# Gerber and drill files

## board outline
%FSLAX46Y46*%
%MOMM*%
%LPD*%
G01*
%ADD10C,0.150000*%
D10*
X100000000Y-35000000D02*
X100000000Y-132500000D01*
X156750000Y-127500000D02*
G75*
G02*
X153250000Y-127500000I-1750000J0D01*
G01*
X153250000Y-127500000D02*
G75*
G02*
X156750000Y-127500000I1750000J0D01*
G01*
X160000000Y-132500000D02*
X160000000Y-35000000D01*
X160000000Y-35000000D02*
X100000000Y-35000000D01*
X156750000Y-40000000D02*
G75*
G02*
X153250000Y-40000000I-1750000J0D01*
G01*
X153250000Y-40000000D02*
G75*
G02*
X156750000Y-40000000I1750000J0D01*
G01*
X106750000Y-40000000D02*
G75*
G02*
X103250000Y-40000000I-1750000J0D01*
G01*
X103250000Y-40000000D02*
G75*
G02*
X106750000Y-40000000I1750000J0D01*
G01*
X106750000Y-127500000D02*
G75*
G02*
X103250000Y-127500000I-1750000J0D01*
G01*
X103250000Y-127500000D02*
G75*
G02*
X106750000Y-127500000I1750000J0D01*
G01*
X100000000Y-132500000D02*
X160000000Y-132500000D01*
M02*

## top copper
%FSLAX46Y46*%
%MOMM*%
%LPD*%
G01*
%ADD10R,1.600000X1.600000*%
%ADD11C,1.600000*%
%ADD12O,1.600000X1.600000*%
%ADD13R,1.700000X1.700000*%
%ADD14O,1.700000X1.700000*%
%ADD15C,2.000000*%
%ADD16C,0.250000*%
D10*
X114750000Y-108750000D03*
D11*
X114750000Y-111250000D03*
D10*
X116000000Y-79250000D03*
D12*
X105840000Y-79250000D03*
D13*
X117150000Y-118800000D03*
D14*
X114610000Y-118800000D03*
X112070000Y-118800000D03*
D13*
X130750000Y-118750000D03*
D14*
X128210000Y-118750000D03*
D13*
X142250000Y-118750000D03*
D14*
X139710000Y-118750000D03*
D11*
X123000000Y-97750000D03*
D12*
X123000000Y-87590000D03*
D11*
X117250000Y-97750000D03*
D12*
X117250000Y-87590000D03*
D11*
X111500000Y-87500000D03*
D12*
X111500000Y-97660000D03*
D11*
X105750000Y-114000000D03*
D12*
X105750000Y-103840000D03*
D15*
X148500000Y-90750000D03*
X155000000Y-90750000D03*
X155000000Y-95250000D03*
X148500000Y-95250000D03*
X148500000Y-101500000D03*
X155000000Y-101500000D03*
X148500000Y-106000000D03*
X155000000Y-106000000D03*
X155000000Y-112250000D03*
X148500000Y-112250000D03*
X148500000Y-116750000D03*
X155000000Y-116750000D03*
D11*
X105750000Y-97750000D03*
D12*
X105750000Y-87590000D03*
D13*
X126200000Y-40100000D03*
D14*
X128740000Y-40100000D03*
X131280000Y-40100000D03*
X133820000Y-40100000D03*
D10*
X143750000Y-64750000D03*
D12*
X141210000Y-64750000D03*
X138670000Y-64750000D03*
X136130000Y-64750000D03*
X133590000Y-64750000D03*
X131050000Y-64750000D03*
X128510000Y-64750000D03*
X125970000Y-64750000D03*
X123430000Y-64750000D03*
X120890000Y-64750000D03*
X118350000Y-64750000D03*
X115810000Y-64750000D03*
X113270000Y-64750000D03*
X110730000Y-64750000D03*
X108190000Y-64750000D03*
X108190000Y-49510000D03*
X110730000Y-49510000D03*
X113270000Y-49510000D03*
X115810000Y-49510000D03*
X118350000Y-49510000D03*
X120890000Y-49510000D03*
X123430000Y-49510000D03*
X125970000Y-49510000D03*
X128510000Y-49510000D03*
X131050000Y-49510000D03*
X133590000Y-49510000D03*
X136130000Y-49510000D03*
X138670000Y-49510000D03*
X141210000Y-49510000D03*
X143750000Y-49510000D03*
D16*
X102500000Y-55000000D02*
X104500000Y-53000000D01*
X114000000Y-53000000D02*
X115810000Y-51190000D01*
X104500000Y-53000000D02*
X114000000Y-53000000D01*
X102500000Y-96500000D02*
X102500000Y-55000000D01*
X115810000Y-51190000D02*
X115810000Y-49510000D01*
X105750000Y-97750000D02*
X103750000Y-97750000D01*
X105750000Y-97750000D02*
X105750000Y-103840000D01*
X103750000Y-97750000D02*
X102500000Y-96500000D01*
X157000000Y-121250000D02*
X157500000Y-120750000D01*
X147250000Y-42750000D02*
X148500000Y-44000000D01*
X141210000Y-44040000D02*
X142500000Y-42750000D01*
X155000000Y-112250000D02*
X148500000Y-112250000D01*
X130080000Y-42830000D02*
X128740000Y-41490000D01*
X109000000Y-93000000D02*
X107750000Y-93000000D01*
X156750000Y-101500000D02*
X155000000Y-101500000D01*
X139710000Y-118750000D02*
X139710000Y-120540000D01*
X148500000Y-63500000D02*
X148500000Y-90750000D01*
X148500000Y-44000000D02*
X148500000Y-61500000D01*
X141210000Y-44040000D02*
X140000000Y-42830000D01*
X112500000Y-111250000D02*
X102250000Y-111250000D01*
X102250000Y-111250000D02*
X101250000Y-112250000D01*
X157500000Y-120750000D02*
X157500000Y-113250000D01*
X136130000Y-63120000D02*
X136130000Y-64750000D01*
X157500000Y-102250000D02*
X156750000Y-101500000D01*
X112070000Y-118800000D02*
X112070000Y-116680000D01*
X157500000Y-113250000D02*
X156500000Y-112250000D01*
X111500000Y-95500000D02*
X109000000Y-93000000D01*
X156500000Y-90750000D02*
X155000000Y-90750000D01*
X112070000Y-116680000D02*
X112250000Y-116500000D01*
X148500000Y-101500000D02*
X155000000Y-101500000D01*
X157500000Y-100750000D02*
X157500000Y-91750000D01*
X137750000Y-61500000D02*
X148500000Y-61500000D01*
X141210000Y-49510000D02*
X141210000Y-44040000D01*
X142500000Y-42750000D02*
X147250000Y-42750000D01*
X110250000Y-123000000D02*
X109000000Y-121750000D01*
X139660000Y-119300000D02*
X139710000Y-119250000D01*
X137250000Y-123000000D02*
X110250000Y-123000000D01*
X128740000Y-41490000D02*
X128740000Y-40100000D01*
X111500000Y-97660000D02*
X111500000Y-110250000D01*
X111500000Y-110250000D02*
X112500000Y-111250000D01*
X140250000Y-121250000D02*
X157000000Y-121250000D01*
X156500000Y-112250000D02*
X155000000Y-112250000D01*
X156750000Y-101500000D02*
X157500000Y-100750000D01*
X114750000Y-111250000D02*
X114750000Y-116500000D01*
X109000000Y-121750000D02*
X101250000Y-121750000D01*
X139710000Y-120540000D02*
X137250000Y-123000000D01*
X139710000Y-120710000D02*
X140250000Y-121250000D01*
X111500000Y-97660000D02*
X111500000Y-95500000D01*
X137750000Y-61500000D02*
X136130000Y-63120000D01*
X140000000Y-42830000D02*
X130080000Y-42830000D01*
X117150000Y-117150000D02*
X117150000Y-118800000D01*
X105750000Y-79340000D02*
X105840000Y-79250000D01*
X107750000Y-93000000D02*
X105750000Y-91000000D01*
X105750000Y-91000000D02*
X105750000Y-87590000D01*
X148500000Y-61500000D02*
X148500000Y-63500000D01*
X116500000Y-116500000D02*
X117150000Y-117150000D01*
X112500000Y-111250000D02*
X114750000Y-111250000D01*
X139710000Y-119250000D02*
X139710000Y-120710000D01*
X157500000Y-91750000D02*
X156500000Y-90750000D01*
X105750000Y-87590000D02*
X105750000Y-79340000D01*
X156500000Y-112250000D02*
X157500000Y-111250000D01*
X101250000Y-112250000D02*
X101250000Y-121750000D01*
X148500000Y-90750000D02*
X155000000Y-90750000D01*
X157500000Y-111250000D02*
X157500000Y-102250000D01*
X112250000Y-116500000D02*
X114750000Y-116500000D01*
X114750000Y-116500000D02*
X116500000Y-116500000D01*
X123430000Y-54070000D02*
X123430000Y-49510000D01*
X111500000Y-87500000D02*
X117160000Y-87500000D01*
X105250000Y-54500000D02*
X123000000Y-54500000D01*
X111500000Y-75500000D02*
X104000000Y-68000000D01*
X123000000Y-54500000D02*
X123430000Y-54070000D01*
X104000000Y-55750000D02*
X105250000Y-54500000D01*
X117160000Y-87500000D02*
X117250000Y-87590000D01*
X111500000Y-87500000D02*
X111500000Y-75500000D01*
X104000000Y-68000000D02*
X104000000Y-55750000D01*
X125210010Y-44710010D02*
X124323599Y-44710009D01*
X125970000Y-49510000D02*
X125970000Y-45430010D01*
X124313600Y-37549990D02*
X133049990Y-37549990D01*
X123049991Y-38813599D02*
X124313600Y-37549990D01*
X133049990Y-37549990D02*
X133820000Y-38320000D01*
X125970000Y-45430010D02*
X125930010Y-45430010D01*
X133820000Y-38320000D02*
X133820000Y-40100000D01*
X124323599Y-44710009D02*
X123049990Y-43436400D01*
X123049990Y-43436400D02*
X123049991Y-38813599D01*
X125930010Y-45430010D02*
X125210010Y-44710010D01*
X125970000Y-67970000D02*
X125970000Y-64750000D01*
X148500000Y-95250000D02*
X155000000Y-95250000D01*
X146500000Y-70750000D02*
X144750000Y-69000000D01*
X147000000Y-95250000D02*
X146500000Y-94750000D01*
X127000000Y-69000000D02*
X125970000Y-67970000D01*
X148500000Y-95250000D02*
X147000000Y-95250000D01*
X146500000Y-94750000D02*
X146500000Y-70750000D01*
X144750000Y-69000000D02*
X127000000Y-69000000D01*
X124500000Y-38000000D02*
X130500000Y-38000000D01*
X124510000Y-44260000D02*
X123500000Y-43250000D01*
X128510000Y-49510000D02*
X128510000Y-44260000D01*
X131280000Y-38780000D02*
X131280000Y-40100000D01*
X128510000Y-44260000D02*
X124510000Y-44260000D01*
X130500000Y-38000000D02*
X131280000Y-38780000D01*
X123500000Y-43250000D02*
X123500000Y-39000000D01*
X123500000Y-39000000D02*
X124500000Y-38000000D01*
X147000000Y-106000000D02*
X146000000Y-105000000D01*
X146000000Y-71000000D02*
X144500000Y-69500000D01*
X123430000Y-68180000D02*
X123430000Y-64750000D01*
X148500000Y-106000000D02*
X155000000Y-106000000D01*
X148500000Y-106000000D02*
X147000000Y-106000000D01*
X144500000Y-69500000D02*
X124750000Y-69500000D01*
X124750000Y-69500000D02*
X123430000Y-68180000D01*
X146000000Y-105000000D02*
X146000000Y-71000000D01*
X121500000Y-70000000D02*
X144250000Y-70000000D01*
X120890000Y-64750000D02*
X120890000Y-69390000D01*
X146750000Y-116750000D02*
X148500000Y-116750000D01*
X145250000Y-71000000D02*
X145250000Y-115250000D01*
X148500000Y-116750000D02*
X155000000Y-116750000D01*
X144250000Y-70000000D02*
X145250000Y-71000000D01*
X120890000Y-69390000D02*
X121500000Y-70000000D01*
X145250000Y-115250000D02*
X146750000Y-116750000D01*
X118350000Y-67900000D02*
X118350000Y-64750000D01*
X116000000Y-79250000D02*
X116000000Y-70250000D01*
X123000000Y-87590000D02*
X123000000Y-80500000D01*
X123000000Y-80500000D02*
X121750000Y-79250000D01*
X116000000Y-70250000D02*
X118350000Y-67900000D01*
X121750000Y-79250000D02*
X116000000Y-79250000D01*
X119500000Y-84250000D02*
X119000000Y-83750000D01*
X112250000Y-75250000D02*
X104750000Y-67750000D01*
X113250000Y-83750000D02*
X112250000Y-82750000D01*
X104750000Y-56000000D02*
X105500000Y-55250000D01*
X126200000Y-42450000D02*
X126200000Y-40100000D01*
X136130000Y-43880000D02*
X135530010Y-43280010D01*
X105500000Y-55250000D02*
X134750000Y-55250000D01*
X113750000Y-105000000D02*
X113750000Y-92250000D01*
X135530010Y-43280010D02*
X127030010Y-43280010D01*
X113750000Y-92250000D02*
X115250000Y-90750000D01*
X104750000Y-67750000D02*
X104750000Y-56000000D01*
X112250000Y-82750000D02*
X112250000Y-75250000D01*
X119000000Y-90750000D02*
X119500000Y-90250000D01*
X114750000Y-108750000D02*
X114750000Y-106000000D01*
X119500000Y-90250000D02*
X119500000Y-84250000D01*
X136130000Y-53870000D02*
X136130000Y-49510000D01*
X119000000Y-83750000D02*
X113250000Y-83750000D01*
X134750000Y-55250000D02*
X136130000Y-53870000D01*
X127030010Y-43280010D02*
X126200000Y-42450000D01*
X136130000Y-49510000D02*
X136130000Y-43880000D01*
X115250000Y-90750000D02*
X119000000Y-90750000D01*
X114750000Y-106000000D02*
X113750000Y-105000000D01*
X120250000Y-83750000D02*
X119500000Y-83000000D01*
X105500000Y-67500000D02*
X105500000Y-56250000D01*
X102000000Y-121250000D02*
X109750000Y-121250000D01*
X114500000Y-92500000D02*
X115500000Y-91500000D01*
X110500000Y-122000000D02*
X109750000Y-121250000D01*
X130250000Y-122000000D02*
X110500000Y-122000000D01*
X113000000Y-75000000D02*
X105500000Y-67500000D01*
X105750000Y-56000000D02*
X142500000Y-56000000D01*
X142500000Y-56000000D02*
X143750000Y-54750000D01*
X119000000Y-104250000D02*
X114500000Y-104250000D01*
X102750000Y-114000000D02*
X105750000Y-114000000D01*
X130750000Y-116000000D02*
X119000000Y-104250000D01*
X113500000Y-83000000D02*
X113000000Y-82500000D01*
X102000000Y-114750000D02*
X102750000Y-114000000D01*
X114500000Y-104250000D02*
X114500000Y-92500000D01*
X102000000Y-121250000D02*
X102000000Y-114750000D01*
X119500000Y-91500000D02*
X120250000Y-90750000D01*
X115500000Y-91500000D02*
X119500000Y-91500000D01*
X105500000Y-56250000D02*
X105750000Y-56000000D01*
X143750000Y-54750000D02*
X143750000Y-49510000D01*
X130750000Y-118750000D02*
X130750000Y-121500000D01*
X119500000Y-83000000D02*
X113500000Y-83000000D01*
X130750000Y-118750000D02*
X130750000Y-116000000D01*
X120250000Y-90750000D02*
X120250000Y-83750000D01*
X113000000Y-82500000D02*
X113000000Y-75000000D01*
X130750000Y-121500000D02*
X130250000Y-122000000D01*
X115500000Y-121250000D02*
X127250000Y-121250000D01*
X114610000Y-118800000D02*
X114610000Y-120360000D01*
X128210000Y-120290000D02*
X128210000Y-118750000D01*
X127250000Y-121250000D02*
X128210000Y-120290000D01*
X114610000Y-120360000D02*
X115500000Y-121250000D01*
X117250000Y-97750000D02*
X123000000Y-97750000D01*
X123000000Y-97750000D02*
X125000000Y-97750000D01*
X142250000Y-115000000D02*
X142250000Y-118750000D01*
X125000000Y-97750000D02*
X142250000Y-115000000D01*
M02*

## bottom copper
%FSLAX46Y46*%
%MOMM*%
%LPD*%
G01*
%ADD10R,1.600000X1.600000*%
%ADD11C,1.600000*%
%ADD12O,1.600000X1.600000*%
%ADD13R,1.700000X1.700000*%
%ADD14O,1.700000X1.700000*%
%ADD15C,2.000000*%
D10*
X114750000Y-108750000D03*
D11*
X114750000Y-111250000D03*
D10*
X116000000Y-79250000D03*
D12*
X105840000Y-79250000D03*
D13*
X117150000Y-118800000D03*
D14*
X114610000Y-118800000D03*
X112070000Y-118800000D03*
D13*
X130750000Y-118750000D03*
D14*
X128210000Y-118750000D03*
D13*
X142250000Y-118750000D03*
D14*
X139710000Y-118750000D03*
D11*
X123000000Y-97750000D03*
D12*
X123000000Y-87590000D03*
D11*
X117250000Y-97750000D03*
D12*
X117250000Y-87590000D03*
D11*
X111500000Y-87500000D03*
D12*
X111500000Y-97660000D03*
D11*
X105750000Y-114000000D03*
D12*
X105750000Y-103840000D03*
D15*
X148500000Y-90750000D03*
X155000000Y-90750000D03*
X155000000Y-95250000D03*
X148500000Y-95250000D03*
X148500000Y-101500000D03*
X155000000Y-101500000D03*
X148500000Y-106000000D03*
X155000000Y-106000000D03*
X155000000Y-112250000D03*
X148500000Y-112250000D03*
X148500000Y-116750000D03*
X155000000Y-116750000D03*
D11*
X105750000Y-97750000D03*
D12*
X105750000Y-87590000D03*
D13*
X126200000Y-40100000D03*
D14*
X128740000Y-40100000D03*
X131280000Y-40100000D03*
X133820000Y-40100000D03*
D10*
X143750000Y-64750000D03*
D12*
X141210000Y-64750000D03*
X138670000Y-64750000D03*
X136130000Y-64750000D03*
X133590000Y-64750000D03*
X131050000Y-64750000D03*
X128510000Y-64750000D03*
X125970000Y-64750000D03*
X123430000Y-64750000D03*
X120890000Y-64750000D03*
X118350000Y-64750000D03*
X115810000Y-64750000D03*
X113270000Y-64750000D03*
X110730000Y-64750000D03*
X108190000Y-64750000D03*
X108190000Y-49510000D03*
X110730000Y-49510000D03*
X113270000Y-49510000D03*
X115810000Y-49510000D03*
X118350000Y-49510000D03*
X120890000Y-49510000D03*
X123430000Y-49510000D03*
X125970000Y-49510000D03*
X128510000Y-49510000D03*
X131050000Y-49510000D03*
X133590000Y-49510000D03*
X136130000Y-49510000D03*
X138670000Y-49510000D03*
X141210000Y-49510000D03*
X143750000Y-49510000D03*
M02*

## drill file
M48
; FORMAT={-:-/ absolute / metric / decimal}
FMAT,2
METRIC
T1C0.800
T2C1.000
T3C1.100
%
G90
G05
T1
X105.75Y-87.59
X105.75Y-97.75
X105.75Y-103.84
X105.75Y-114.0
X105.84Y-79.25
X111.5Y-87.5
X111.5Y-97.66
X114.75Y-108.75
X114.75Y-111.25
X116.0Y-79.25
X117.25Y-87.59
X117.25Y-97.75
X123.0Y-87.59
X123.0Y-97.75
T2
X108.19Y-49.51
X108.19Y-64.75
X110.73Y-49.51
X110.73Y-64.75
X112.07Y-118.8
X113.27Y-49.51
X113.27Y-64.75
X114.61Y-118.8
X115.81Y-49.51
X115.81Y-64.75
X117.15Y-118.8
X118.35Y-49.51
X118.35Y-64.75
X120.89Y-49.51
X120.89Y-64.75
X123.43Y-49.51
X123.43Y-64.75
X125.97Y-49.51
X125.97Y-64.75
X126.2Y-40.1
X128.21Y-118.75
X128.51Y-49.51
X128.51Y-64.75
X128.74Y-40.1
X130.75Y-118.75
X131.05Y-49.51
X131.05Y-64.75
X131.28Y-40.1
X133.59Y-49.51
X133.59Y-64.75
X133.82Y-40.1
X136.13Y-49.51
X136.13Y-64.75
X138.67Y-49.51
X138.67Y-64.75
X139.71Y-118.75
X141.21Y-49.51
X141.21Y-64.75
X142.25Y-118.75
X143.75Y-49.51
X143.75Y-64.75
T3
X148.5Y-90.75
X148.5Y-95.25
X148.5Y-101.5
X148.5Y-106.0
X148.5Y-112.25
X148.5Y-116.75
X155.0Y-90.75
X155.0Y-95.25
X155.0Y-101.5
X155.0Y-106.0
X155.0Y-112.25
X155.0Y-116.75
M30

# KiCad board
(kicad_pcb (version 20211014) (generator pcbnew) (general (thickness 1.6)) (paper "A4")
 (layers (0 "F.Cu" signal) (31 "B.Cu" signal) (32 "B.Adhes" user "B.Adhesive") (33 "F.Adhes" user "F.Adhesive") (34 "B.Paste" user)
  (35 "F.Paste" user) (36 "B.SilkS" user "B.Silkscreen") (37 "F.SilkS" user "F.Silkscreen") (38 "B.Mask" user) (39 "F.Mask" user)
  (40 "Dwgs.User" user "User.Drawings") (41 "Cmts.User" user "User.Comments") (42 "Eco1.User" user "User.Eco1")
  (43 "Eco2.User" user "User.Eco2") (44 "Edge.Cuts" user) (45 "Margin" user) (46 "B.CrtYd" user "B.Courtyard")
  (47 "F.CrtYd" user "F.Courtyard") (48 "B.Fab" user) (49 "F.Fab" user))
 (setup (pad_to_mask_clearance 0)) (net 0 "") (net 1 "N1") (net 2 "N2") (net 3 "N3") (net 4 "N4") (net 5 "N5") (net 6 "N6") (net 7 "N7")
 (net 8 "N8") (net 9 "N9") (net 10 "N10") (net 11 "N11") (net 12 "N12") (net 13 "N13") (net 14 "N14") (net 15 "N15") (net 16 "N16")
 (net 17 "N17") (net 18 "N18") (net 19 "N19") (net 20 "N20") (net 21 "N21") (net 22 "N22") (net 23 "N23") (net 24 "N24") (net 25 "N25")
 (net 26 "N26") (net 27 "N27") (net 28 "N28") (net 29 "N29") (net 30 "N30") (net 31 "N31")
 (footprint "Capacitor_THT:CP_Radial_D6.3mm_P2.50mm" (layer "F.Cu") (at 114.75 108.75 -90)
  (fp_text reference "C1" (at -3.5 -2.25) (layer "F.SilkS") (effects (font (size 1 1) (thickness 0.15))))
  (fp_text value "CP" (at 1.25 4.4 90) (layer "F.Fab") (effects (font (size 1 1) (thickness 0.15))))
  (pad "1" thru_hole rect locked (at 0 0 270) (size 1.6 1.6) (drill 0.8) (layers *.Cu *.Mask) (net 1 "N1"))
  (pad "2" thru_hole circle locked (at 2.5 0 270) (size 1.6 1.6) (drill 0.8) (layers *.Cu *.Mask) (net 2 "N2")))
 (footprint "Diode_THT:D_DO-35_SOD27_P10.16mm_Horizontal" (layer "F.Cu") (at 116 79.25 180)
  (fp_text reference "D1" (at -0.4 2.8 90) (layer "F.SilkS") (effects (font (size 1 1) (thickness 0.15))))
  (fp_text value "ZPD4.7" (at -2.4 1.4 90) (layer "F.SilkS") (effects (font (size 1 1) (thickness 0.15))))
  (pad "1" thru_hole rect locked (at 0 0 180) (size 1.6 1.6) (drill 0.8) (layers *.Cu *.Mask) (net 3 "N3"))
  (pad "2" thru_hole oval locked (at 10.16 0 180) (size 1.6 1.6) (drill 0.8) (layers *.Cu *.Mask) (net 2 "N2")))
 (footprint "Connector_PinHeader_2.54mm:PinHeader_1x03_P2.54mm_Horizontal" (layer "F.Cu") (at 117.15 118.8 -90)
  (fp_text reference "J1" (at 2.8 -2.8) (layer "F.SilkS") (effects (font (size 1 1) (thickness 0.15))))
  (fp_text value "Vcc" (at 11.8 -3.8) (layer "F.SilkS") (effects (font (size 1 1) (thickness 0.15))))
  (pad "1" thru_hole rect locked (at 0 0 270) (size 1.7 1.7) (drill 1) (layers *.Cu *.Mask) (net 2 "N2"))
  (pad "2" thru_hole oval locked (at 0 2.54 270) (size 1.7 1.7) (drill 1) (layers *.Cu *.Mask) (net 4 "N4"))
  (pad "3" thru_hole oval locked (at 0 5.08 270) (size 1.7 1.7) (drill 1) (layers *.Cu *.Mask) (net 2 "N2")))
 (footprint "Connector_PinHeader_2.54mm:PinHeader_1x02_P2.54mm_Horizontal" (layer "F.Cu") (at 130.75 118.75 -90)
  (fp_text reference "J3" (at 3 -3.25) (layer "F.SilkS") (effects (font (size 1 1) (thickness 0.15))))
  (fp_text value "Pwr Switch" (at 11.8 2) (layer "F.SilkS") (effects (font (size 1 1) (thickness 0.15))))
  (pad "1" thru_hole rect locked (at 0 0 270) (size 1.7 1.7) (drill 1) (layers *.Cu *.Mask) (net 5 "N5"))
  (pad "2" thru_hole oval locked (at 0 2.54 270) (size 1.7 1.7) (drill 1) (layers *.Cu *.Mask) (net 4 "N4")))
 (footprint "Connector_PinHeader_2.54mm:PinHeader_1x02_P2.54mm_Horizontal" (layer "F.Cu") (at 142.25 118.75 -90)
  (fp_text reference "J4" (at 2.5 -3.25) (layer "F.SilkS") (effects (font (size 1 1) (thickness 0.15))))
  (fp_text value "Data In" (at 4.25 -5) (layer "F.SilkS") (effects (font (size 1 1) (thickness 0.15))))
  (pad "1" thru_hole rect locked (at 0 0 270) (size 1.7 1.7) (drill 1) (layers *.Cu *.Mask) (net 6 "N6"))
  (pad "2" thru_hole oval locked (at 0 2.54 270) (size 1.7 1.7) (drill 1) (layers *.Cu *.Mask) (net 2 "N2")))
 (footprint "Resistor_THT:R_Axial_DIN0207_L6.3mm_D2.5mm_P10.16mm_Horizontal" (layer "F.Cu") (at 123 97.75 90)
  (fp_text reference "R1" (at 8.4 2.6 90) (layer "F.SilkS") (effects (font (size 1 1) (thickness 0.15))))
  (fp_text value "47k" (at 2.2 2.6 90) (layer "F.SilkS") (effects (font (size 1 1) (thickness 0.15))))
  (pad "1" thru_hole circle locked (at 0 0 90) (size 1.6 1.6) (drill 0.8) (layers *.Cu *.Mask) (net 6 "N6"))
  (pad "2" thru_hole oval locked (at 10.16 0 90) (size 1.6 1.6) (drill 0.8) (layers *.Cu *.Mask) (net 3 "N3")))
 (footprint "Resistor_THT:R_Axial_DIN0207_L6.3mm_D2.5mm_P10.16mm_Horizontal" (layer "F.Cu") (at 117.25 97.75 90)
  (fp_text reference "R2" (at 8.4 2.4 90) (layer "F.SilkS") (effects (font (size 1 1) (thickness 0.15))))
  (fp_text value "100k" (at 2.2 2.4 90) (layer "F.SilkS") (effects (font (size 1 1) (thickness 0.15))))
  (pad "1" thru_hole circle locked (at 0 0 90) (size 1.6 1.6) (drill 0.8) (layers *.Cu *.Mask) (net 6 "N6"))
  (pad "2" thru_hole oval locked (at 10.16 0 90) (size 1.6 1.6) (drill 0.8) (layers *.Cu *.Mask) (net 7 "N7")))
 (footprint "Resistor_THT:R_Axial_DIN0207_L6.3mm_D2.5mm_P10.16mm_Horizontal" (layer "F.Cu") (at 111.5 87.5 -90)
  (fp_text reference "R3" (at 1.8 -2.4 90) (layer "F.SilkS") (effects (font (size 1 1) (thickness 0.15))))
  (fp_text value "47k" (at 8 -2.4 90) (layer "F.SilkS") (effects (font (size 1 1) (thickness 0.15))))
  (pad "1" thru_hole circle locked (at 0 0 270) (size 1.6 1.6) (drill 0.8) (layers *.Cu *.Mask) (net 7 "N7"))
  (pad "2" thru_hole oval locked (at 10.16 0 270) (size 1.6 1.6) (drill 0.8) (layers *.Cu *.Mask) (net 2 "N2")))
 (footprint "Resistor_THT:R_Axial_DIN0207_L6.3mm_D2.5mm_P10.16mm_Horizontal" (layer "F.Cu") (at 105.75 114 90)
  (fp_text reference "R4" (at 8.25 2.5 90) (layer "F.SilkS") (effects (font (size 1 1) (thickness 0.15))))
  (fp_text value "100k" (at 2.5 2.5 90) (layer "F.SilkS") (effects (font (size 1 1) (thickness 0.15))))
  (pad "1" thru_hole circle locked (at 0 0 90) (size 1.6 1.6) (drill 0.8) (layers *.Cu *.Mask) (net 5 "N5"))
  (pad "2" thru_hole oval locked (at 10.16 0 90) (size 1.6 1.6) (drill 0.8) (layers *.Cu *.Mask) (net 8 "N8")))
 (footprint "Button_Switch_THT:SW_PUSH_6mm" (layer "F.Cu") (at 148.5 90.75)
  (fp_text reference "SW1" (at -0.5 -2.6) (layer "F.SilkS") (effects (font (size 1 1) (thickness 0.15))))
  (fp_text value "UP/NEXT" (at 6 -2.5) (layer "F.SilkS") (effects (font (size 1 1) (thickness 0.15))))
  (pad "1" thru_hole circle locked (at 0 0 90) (size 2 2) (drill 1.1) (layers *.Cu *.Mask) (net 2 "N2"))
  (pad "1" thru_hole circle locked (at 6.5 0 90) (size 2 2) (drill 1.1) (layers *.Cu *.Mask) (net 2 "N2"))
  (pad "2" thru_hole circle locked (at 6.5 4.5 90) (size 2 2) (drill 1.1) (layers *.Cu *.Mask) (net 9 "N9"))
  (pad "2" thru_hole circle locked (at 0 4.5 90) (size 2 2) (drill 1.1) (layers *.Cu *.Mask) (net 9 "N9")))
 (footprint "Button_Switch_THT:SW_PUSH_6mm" (layer "F.Cu") (at 148.5 101.5)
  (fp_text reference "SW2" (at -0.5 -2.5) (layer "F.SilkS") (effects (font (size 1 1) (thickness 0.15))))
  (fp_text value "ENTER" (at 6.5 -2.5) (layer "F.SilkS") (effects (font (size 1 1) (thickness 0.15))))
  (pad "1" thru_hole circle locked (at 0 0 90) (size 2 2) (drill 1.1) (layers *.Cu *.Mask) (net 2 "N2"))
  (pad "1" thru_hole circle locked (at 6.5 0 90) (size 2 2) (drill 1.1) (layers *.Cu *.Mask) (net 2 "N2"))
  (pad "2" thru_hole circle locked (at 0 4.5 90) (size 2 2) (drill 1.1) (layers *.Cu *.Mask) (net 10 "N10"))
  (pad "2" thru_hole circle locked (at 6.5 4.5 90) (size 2 2) (drill 1.1) (layers *.Cu *.Mask) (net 10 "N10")))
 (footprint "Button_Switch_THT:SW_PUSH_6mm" (layer "F.Cu") (at 148.5 112.25)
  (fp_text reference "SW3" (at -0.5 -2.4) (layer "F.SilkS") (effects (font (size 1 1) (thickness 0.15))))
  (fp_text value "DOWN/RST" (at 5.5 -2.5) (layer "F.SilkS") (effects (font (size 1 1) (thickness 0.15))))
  (pad "1" thru_hole circle locked (at 6.5 0 90) (size 2 2) (drill 1.1) (layers *.Cu *.Mask) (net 2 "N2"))
  (pad "1" thru_hole circle locked (at 0 0 90) (size 2 2) (drill 1.1) (layers *.Cu *.Mask) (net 2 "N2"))
  (pad "2" thru_hole circle locked (at 0 4.5 90) (size 2 2) (drill 1.1) (layers *.Cu *.Mask) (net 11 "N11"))
  (pad "2" thru_hole circle locked (at 6.5 4.5 90) (size 2 2) (drill 1.1) (layers *.Cu *.Mask) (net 11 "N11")))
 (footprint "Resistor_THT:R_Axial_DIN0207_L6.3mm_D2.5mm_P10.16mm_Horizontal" (layer "F.Cu") (at 105.75 97.75 90)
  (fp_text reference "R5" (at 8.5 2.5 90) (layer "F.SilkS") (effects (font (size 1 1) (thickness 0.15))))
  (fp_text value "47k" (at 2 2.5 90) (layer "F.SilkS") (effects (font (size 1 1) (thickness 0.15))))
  (pad "1" thru_hole circle locked (at 0 0 90) (size 1.6 1.6) (drill 0.8) (layers *.Cu *.Mask) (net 8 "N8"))
  (pad "2" thru_hole oval locked (at 10.16 0 90) (size 1.6 1.6) (drill 0.8) (layers *.Cu *.Mask) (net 2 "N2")))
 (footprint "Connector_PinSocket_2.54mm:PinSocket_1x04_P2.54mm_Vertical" (layer "F.Cu") (at 126.2 40.1 90)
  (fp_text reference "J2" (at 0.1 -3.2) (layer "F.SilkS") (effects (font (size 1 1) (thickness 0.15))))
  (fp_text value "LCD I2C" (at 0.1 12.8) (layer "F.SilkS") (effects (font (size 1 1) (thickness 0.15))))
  (pad "1" thru_hole rect locked (at 0 0 90) (size 1.7 1.7) (drill 1) (layers *.Cu *.Mask) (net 1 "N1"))
  (pad "2" thru_hole oval locked (at 0 2.54 90) (size 1.7 1.7) (drill 1) (layers *.Cu *.Mask) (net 2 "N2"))
  (pad "3" thru_hole oval locked (at 0 5.08 90) (size 1.7 1.7) (drill 1) (layers *.Cu *.Mask) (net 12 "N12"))
  (pad "4" thru_hole oval locked (at 0 7.62 90) (size 1.7 1.7) (drill 1) (layers *.Cu *.Mask) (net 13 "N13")))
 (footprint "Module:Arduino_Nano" (layer "B.Cu") (at 143.75 64.75 90)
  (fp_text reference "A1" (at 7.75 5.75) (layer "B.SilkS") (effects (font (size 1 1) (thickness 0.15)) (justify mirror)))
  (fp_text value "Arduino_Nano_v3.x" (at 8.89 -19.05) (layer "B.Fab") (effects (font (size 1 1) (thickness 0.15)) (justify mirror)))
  (pad "1" thru_hole rect locked (at 0 0 90) (size 1.6 1.6) (drill 1) (layers *.Cu *.Mask) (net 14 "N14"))
  (pad "2" thru_hole oval locked (at 0 -2.54 90) (size 1.6 1.6) (drill 1) (layers *.Cu *.Mask) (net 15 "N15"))
  (pad "3" thru_hole oval locked (at 0 -5.08 90) (size 1.6 1.6) (drill 1) (layers *.Cu *.Mask) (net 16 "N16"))
  (pad "4" thru_hole oval locked (at 0 -7.62 90) (size 1.6 1.6) (drill 1) (layers *.Cu *.Mask) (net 2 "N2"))
  (pad "5" thru_hole oval locked (at 0 -10.16 90) (size 1.6 1.6) (drill 1) (layers *.Cu *.Mask) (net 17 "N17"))
  (pad "6" thru_hole oval locked (at 0 -12.7 90) (size 1.6 1.6) (drill 1) (layers *.Cu *.Mask) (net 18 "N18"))
  (pad "7" thru_hole oval locked (at 0 -15.24 90) (size 1.6 1.6) (drill 1) (layers *.Cu *.Mask) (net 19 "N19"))
  (pad "8" thru_hole oval locked (at 0 -17.78 90) (size 1.6 1.6) (drill 1) (layers *.Cu *.Mask) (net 9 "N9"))
  (pad "9" thru_hole oval locked (at 0 -20.32 90) (size 1.6 1.6) (drill 1) (layers *.Cu *.Mask) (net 10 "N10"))
  (pad "10" thru_hole oval locked (at 0 -22.86 90) (size 1.6 1.6) (drill 1) (layers *.Cu *.Mask) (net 11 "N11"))
  (pad "11" thru_hole oval locked (at 0 -25.4 90) (size 1.6 1.6) (drill 1) (layers *.Cu *.Mask) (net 3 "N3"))
  (pad "12" thru_hole oval locked (at 0 -27.94 90) (size 1.6 1.6) (drill 1) (layers *.Cu *.Mask) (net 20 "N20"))
  (pad "13" thru_hole oval locked (at 0 -30.48 90) (size 1.6 1.6) (drill 1) (layers *.Cu *.Mask) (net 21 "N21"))
  (pad "14" thru_hole oval locked (at 0 -33.02 90) (size 1.6 1.6) (drill 1) (layers *.Cu *.Mask) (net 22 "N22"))
  (pad "15" thru_hole oval locked (at 0 -35.56 90) (size 1.6 1.6) (drill 1) (layers *.Cu *.Mask) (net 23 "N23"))
  (pad "16" thru_hole oval locked (at 15.24 -35.56 90) (size 1.6 1.6) (drill 1) (layers *.Cu *.Mask) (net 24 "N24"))
  (pad "17" thru_hole oval locked (at 15.24 -33.02 90) (size 1.6 1.6) (drill 1) (layers *.Cu *.Mask) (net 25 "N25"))
  (pad "18" thru_hole oval locked (at 15.24 -30.48 90) (size 1.6 1.6) (drill 1) (layers *.Cu *.Mask) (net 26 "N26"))
  (pad "19" thru_hole oval locked (at 15.24 -27.94 90) (size 1.6 1.6) (drill 1) (layers *.Cu *.Mask) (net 8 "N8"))
  (pad "20" thru_hole oval locked (at 15.24 -25.4 90) (size 1.6 1.6) (drill 1) (layers *.Cu *.Mask) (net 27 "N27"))
  (pad "21" thru_hole oval locked (at 15.24 -22.86 90) (size 1.6 1.6) (drill 1) (layers *.Cu *.Mask) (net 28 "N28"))
  (pad "22" thru_hole oval locked (at 15.24 -20.32 90) (size 1.6 1.6) (drill 1) (layers *.Cu *.Mask) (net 7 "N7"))
  (pad "23" thru_hole oval locked (at 15.24 -17.78 90) (size 1.6 1.6) (drill 1) (layers *.Cu *.Mask) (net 13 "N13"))
  (pad "24" thru_hole oval locked (at 15.24 -15.24 90) (size 1.6 1.6) (drill 1) (layers *.Cu *.Mask) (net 12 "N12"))
  (pad "25" thru_hole oval locked (at 15.24 -12.7 90) (size 1.6 1.6) (drill 1) (layers *.Cu *.Mask) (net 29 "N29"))
  (pad "26" thru_hole oval locked (at 15.24 -10.16 90) (size 1.6 1.6) (drill 1) (layers *.Cu *.Mask) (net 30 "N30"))
  (pad "27" thru_hole oval locked (at 15.24 -7.62 90) (size 1.6 1.6) (drill 1) (layers *.Cu *.Mask) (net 1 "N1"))
  (pad "28" thru_hole oval locked (at 15.24 -5.08 90) (size 1.6 1.6) (drill 1) (layers *.Cu *.Mask) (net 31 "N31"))
  (pad "29" thru_hole oval locked (at 15.24 -2.54 90) (size 1.6 1.6) (drill 1) (layers *.Cu *.Mask) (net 2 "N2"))
  (pad "30" thru_hole oval locked (at 15.24 0 90) (size 1.6 1.6) (drill 1) (layers *.Cu *.Mask) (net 5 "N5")))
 (gr_line (start 100 35) (end 100 132.5) (layer "Edge.Cuts") (width 0.15))
 (gr_circle (center 155 127.5) (end 156.75 127.5) (layer "Edge.Cuts") (width 0.15) (fill none))
 (gr_line (start 160 132.5) (end 160 35) (layer "Edge.Cuts") (width 0.15))
 (gr_line (start 160 35) (end 100 35) (layer "Edge.Cuts") (width 0.15))
 (gr_circle (center 155 40) (end 156.75 40) (layer "Edge.Cuts") (width 0.15) (fill none))
 (gr_circle (center 105 40) (end 106.75 40) (layer "Edge.Cuts") (width 0.15) (fill none))
 (gr_circle (center 105 127.5) (end 106.75 127.5) (layer "Edge.Cuts") (width 0.15) (fill none))
 (gr_line (start 100 132.5) (end 160 132.5) (layer "Edge.Cuts") (width 0.15))
 (segment (start 102.5 55) (end 104.5 53) (width 0.25) (layer "F.Cu") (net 8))
 (segment (start 114 53) (end 115.81 51.19) (width 0.25) (layer "F.Cu") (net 8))
 (segment (start 104.5 53) (end 114 53) (width 0.25) (layer "F.Cu") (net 8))
 (segment (start 102.5 96.5) (end 102.5 55) (width 0.25) (layer "F.Cu") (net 8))
 (segment (start 115.81 51.19) (end 115.81 49.51) (width 0.25) (layer "F.Cu") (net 8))
 (segment (start 105.75 97.75) (end 103.75 97.75) (width 0.25) (layer "F.Cu") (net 8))
 (segment (start 105.75 97.75) (end 105.75 103.84) (width 0.25) (layer "F.Cu") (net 8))
 (segment (start 103.75 97.75) (end 102.5 96.5) (width 0.25) (layer "F.Cu") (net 8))
 (segment (start 157 121.25) (end 157.5 120.75) (width 0.25) (layer "F.Cu") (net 2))
 (segment (start 147.25 42.75) (end 148.5 44) (width 0.25) (layer "F.Cu") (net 2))
 (segment (start 141.21 44.04) (end 142.5 42.75) (width 0.25) (layer "F.Cu") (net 2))
 (segment (start 155 112.25) (end 148.5 112.25) (width 0.25) (layer "F.Cu") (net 2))
 (segment (start 130.08 42.83) (end 128.74 41.49) (width 0.25) (layer "F.Cu") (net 2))
 (segment (start 109 93) (end 107.75 93) (width 0.25) (layer "F.Cu") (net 2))
 (segment (start 156.75 101.5) (end 155 101.5) (width 0.25) (layer "F.Cu") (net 2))
 (segment (start 139.71 118.75) (end 139.71 120.54) (width 0.25) (layer "F.Cu") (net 2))
 (segment (start 148.5 63.5) (end 148.5 90.75) (width 0.25) (layer "F.Cu") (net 2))
 (segment (start 148.5 44) (end 148.5 61.5) (width 0.25) (layer "F.Cu") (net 2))
 (segment (start 141.21 44.04) (end 140 42.83) (width 0.25) (layer "F.Cu") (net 2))
 (segment (start 112.5 111.25) (end 102.25 111.25) (width 0.25) (layer "F.Cu") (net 2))
 (segment (start 102.25 111.25) (end 101.25 112.25) (width 0.25) (layer "F.Cu") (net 2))
 (segment (start 157.5 120.75) (end 157.5 113.25) (width 0.25) (layer "F.Cu") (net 2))
 (segment (start 136.13 63.12) (end 136.13 64.75) (width 0.25) (layer "F.Cu") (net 2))
 (segment (start 157.5 102.25) (end 156.75 101.5) (width 0.25) (layer "F.Cu") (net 2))
 (segment (start 112.07 118.8) (end 112.07 116.68) (width 0.25) (layer "F.Cu") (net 2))
 (segment (start 157.5 113.25) (end 156.5 112.25) (width 0.25) (layer "F.Cu") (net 2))
 (segment (start 111.5 95.5) (end 109 93) (width 0.25) (layer "F.Cu") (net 2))
 (segment (start 156.5 90.75) (end 155 90.75) (width 0.25) (layer "F.Cu") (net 2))
 (segment (start 112.07 116.68) (end 112.25 116.5) (width 0.25) (layer "F.Cu") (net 2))
 (segment (start 148.5 101.5) (end 155 101.5) (width 0.25) (layer "F.Cu") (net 2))
 (segment (start 157.5 100.75) (end 157.5 91.75) (width 0.25) (layer "F.Cu") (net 2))
 (segment (start 137.75 61.5) (end 148.5 61.5) (width 0.25) (layer "F.Cu") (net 2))
 (segment (start 141.21 49.51) (end 141.21 44.04) (width 0.25) (layer "F.Cu") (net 2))
 (segment (start 142.5 42.75) (end 147.25 42.75) (width 0.25) (layer "F.Cu") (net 2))
 (segment (start 110.25 123) (end 109 121.75) (width 0.25) (layer "F.Cu") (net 2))
 (segment (start 139.66 119.3) (end 139.71 119.25) (width 0.25) (layer "F.Cu") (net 2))
 (segment (start 137.25 123) (end 110.25 123) (width 0.25) (layer "F.Cu") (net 2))
 (segment (start 128.74 41.49) (end 128.74 40.1) (width 0.25) (layer "F.Cu") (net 2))
 (segment (start 111.5 97.66) (end 111.5 110.25) (width 0.25) (layer "F.Cu") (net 2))
 (segment (start 111.5 110.25) (end 112.5 111.25) (width 0.25) (layer "F.Cu") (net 2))
 (segment (start 140.25 121.25) (end 157 121.25) (width 0.25) (layer "F.Cu") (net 2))
 (segment (start 156.5 112.25) (end 155 112.25) (width 0.25) (layer "F.Cu") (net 2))
 (segment (start 156.75 101.5) (end 157.5 100.75) (width 0.25) (layer "F.Cu") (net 2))
 (segment (start 114.75 111.25) (end 114.75 116.5) (width 0.25) (layer "F.Cu") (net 2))
 (segment (start 109 121.75) (end 101.25 121.75) (width 0.25) (layer "F.Cu") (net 2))
 (segment (start 139.71 120.54) (end 137.25 123) (width 0.25) (layer "F.Cu") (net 2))
 (segment (start 139.71 120.71) (end 140.25 121.25) (width 0.25) (layer "F.Cu") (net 2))
 (segment (start 111.5 97.66) (end 111.5 95.5) (width 0.25) (layer "F.Cu") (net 2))
 (segment (start 137.75 61.5) (end 136.13 63.12) (width 0.25) (layer "F.Cu") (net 2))
 (segment (start 140 42.83) (end 130.08 42.83) (width 0.25) (layer "F.Cu") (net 2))
 (segment (start 117.15 117.15) (end 117.15 118.8) (width 0.25) (layer "F.Cu") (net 2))
 (segment (start 105.75 79.34) (end 105.84 79.25) (width 0.25) (layer "F.Cu") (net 2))
 (segment (start 107.75 93) (end 105.75 91) (width 0.25) (layer "F.Cu") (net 2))
 (segment (start 105.75 91) (end 105.75 87.59) (width 0.25) (layer "F.Cu") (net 2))
 (segment (start 148.5 61.5) (end 148.5 63.5) (width 0.25) (layer "F.Cu") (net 2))
 (segment (start 116.5 116.5) (end 117.15 117.15) (width 0.25) (layer "F.Cu") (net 2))
 (segment (start 112.5 111.25) (end 114.75 111.25) (width 0.25) (layer "F.Cu") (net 2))
 (segment (start 139.71 119.25) (end 139.71 120.71) (width 0.25) (layer "F.Cu") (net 2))
 (segment (start 157.5 91.75) (end 156.5 90.75) (width 0.25) (layer "F.Cu") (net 2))
 (segment (start 105.75 87.59) (end 105.75 79.34) (width 0.25) (layer "F.Cu") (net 2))
 (segment (start 156.5 112.25) (end 157.5 111.25) (width 0.25) (layer "F.Cu") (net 2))
 (segment (start 101.25 112.25) (end 101.25 121.75) (width 0.25) (layer "F.Cu") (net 2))
 (segment (start 148.5 90.75) (end 155 90.75) (width 0.25) (layer "F.Cu") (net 2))
 (segment (start 157.5 111.25) (end 157.5 102.25) (width 0.25) (layer "F.Cu") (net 2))
 (segment (start 112.25 116.5) (end 114.75 116.5) (width 0.25) (layer "F.Cu") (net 2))
 (segment (start 114.75 116.5) (end 116.5 116.5) (width 0.25) (layer "F.Cu") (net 2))
 (segment (start 123.43 54.07) (end 123.43 49.51) (width 0.25) (layer "F.Cu") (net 7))
 (segment (start 111.5 87.5) (end 117.16 87.5) (width 0.25) (layer "F.Cu") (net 7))
 (segment (start 105.25 54.5) (end 123 54.5) (width 0.25) (layer "F.Cu") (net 7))
 (segment (start 111.5 75.5) (end 104 68) (width 0.25) (layer "F.Cu") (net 7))
 (segment (start 123 54.5) (end 123.43 54.07) (width 0.25) (layer "F.Cu") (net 7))
 (segment (start 104 55.75) (end 105.25 54.5) (width 0.25) (layer "F.Cu") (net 7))
 (segment (start 117.16 87.5) (end 117.25 87.59) (width 0.25) (layer "F.Cu") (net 7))
 (segment (start 111.5 87.5) (end 111.5 75.5) (width 0.25) (layer "F.Cu") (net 7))
 (segment (start 104 68) (end 104 55.75) (width 0.25) (layer "F.Cu") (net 7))
 (segment (start 125.21001 44.71001) (end 124.323599 44.710009) (width 0.25) (layer "F.Cu") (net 13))
 (segment (start 125.97 49.51) (end 125.97 45.43001) (width 0.25) (layer "F.Cu") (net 13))
 (segment (start 124.3136 37.54999) (end 133.04999 37.54999) (width 0.25) (layer "F.Cu") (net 13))
 (segment (start 123.049991 38.813599) (end 124.3136 37.54999) (width 0.25) (layer "F.Cu") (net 13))
 (segment (start 133.04999 37.54999) (end 133.82 38.32) (width 0.25) (layer "F.Cu") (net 13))
 (segment (start 125.97 45.43001) (end 125.93001 45.43001) (width 0.25) (layer "F.Cu") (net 13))
 (segment (start 133.82 38.32) (end 133.82 40.1) (width 0.25) (layer "F.Cu") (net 13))
 (segment (start 124.323599 44.710009) (end 123.04999 43.4364) (width 0.25) (layer "F.Cu") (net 13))
 (segment (start 123.04999 43.4364) (end 123.049991 38.813599) (width 0.25) (layer "F.Cu") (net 13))
 (segment (start 125.93001 45.43001) (end 125.21001 44.71001) (width 0.25) (layer "F.Cu") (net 13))
 (segment (start 125.97 67.97) (end 125.97 64.75) (width 0.25) (layer "F.Cu") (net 9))
 (segment (start 148.5 95.25) (end 155 95.25) (width 0.25) (layer "F.Cu") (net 9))
 (segment (start 146.5 70.75) (end 144.75 69) (width 0.25) (layer "F.Cu") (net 9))
 (segment (start 147 95.25) (end 146.5 94.75) (width 0.25) (layer "F.Cu") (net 9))
 (segment (start 127 69) (end 125.97 67.97) (width 0.25) (layer "F.Cu") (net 9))
 (segment (start 148.5 95.25) (end 147 95.25) (width 0.25) (layer "F.Cu") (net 9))
 (segment (start 146.5 94.75) (end 146.5 70.75) (width 0.25) (layer "F.Cu") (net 9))
 (segment (start 144.75 69) (end 127 69) (width 0.25) (layer "F.Cu") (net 9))
 (segment (start 124.5 38) (end 130.5 38) (width 0.25) (layer "F.Cu") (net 12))
 (segment (start 124.51 44.26) (end 123.5 43.25) (width 0.25) (layer "F.Cu") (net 12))
 (segment (start 128.51 49.51) (end 128.51 44.26) (width 0.25) (layer "F.Cu") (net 12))
 (segment (start 131.28 38.78) (end 131.28 40.1) (width 0.25) (layer "F.Cu") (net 12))
 (segment (start 128.51 44.26) (end 124.51 44.26) (width 0.25) (layer "F.Cu") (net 12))
 (segment (start 130.5 38) (end 131.28 38.78) (width 0.25) (layer "F.Cu") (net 12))
 (segment (start 123.5 43.25) (end 123.5 39) (width 0.25) (layer "F.Cu") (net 12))
 (segment (start 123.5 39) (end 124.5 38) (width 0.25) (layer "F.Cu") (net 12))
 (segment (start 147 106) (end 146 105) (width 0.25) (layer "F.Cu") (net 10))
 (segment (start 146 71) (end 144.5 69.5) (width 0.25) (layer "F.Cu") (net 10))
 (segment (start 123.43 68.18) (end 123.43 64.75) (width 0.25) (layer "F.Cu") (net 10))
 (segment (start 148.5 106) (end 155 106) (width 0.25) (layer "F.Cu") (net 10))
 (segment (start 148.5 106) (end 147 106) (width 0.25) (layer "F.Cu") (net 10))
 (segment (start 144.5 69.5) (end 124.75 69.5) (width 0.25) (layer "F.Cu") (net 10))
 (segment (start 124.75 69.5) (end 123.43 68.18) (width 0.25) (layer "F.Cu") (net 10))
 (segment (start 146 105) (end 146 71) (width 0.25) (layer "F.Cu") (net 10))
 (segment (start 121.5 70) (end 144.25 70) (width 0.25) (layer "F.Cu") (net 11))
 (segment (start 120.89 64.75) (end 120.89 69.39) (width 0.25) (layer "F.Cu") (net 11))
 (segment (start 146.75 116.75) (end 148.5 116.75) (width 0.25) (layer "F.Cu") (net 11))
 (segment (start 145.25 71) (end 145.25 115.25) (width 0.25) (layer "F.Cu") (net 11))
 (segment (start 148.5 116.75) (end 155 116.75) (width 0.25) (layer "F.Cu") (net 11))
 (segment (start 144.25 70) (end 145.25 71) (width 0.25) (layer "F.Cu") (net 11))
 (segment (start 120.89 69.39) (end 121.5 70) (width 0.25) (layer "F.Cu") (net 11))
 (segment (start 145.25 115.25) (end 146.75 116.75) (width 0.25) (layer "F.Cu") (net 11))
 (segment (start 118.35 67.9) (end 118.35 64.75) (width 0.25) (layer "F.Cu") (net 3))
 (segment (start 116 79.25) (end 116 70.25) (width 0.25) (layer "F.Cu") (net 3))
 (segment (start 123 87.59) (end 123 80.5) (width 0.25) (layer "F.Cu") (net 3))
 (segment (start 123 80.5) (end 121.75 79.25) (width 0.25) (layer "F.Cu") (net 3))
 (segment (start 116 70.25) (end 118.35 67.9) (width 0.25) (layer "F.Cu") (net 3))
 (segment (start 121.75 79.25) (end 116 79.25) (width 0.25) (layer "F.Cu") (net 3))
 (segment (start 119.5 84.25) (end 119 83.75) (width 0.25) (layer "F.Cu") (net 1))
 (segment (start 112.25 75.25) (end 104.75 67.75) (width 0.25) (layer "F.Cu") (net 1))
 (segment (start 113.25 83.75) (end 112.25 82.75) (width 0.25) (layer "F.Cu") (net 1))
 (segment (start 104.75 56) (end 105.5 55.25) (width 0.25) (layer "F.Cu") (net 1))
 (segment (start 126.2 42.45) (end 126.2 40.1) (width 0.25) (layer "F.Cu") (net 1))
 (segment (start 136.13 43.88) (end 135.53001 43.28001) (width 0.25) (layer "F.Cu") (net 1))
 (segment (start 105.5 55.25) (end 134.75 55.25) (width 0.25) (layer "F.Cu") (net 1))
 (segment (start 113.75 105) (end 113.75 92.25) (width 0.25) (layer "F.Cu") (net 1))
 (segment (start 135.53001 43.28001) (end 127.03001 43.28001) (width 0.25) (layer "F.Cu") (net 1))
 (segment (start 113.75 92.25) (end 115.25 90.75) (width 0.25) (layer "F.Cu") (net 1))
 (segment (start 104.75 67.75) (end 104.75 56) (width 0.25) (layer "F.Cu") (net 1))
 (segment (start 112.25 82.75) (end 112.25 75.25) (width 0.25) (layer "F.Cu") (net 1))
 (segment (start 119 90.75) (end 119.5 90.25) (width 0.25) (layer "F.Cu") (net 1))
 (segment (start 114.75 108.75) (end 114.75 106) (width 0.25) (layer "F.Cu") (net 1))
 (segment (start 119.5 90.25) (end 119.5 84.25) (width 0.25) (layer "F.Cu") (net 1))
 (segment (start 136.13 53.87) (end 136.13 49.51) (width 0.25) (layer "F.Cu") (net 1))
 (segment (start 119 83.75) (end 113.25 83.75) (width 0.25) (layer "F.Cu") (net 1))
 (segment (start 134.75 55.25) (end 136.13 53.87) (width 0.25) (layer "F.Cu") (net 1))
 (segment (start 127.03001 43.28001) (end 126.2 42.45) (width 0.25) (layer "F.Cu") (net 1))
 (segment (start 136.13 49.51) (end 136.13 43.88) (width 0.25) (layer "F.Cu") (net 1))
 (segment (start 115.25 90.75) (end 119 90.75) (width 0.25) (layer "F.Cu") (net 1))
 (segment (start 114.75 106) (end 113.75 105) (width 0.25) (layer "F.Cu") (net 1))
 (segment (start 120.25 83.75) (end 119.5 83) (width 0.25) (layer "F.Cu") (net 5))
 (segment (start 105.5 67.5) (end 105.5 56.25) (width 0.25) (layer "F.Cu") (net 5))
 (segment (start 102 121.25) (end 109.75 121.25) (width 0.25) (layer "F.Cu") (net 5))
 (segment (start 114.5 92.5) (end 115.5 91.5) (width 0.25) (layer "F.Cu") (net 5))
 (segment (start 110.5 122) (end 109.75 121.25) (width 0.25) (layer "F.Cu") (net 5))
 (segment (start 130.25 122) (end 110.5 122) (width 0.25) (layer "F.Cu") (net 5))
 (segment (start 113 75) (end 105.5 67.5) (width 0.25) (layer "F.Cu") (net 5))
 (segment (start 105.75 56) (end 142.5 56) (width 0.25) (layer "F.Cu") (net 5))
 (segment (start 142.5 56) (end 143.75 54.75) (width 0.25) (layer "F.Cu") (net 5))
 (segment (start 119 104.25) (end 114.5 104.25) (width 0.25) (layer "F.Cu") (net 5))
 (segment (start 102.75 114) (end 105.75 114) (width 0.25) (layer "F.Cu") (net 5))
 (segment (start 130.75 116) (end 119 104.25) (width 0.25) (layer "F.Cu") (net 5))
 (segment (start 113.5 83) (end 113 82.5) (width 0.25) (layer "F.Cu") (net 5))
 (segment (start 102 114.75) (end 102.75 114) (width 0.25) (layer "F.Cu") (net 5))
 (segment (start 114.5 104.25) (end 114.5 92.5) (width 0.25) (layer "F.Cu") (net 5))
 (segment (start 102 121.25) (end 102 114.75) (width 0.25) (layer "F.Cu") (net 5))
 (segment (start 119.5 91.5) (end 120.25 90.75) (width 0.25) (layer "F.Cu") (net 5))
 (segment (start 115.5 91.5) (end 119.5 91.5) (width 0.25) (layer "F.Cu") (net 5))
 (segment (start 105.5 56.25) (end 105.75 56) (width 0.25) (layer "F.Cu") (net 5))
 (segment (start 143.75 54.75) (end 143.75 49.51) (width 0.25) (layer "F.Cu") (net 5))
 (segment (start 130.75 118.75) (end 130.75 121.5) (width 0.25) (layer "F.Cu") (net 5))
 (segment (start 119.5 83) (end 113.5 83) (width 0.25) (layer "F.Cu") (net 5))
 (segment (start 130.75 118.75) (end 130.75 116) (width 0.25) (layer "F.Cu") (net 5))
 (segment (start 120.25 90.75) (end 120.25 83.75) (width 0.25) (layer "F.Cu") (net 5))
 (segment (start 113 82.5) (end 113 75) (width 0.25) (layer "F.Cu") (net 5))
 (segment (start 130.75 121.5) (end 130.25 122) (width 0.25) (layer "F.Cu") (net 5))
 (segment (start 115.5 121.25) (end 127.25 121.25) (width 0.25) (layer "F.Cu") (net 4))
 (segment (start 114.61 118.8) (end 114.61 120.36) (width 0.25) (layer "F.Cu") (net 4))
 (segment (start 128.21 120.29) (end 128.21 118.75) (width 0.25) (layer "F.Cu") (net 4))
 (segment (start 127.25 121.25) (end 128.21 120.29) (width 0.25) (layer "F.Cu") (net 4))
 (segment (start 114.61 120.36) (end 115.5 121.25) (width 0.25) (layer "F.Cu") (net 4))
 (segment (start 117.25 97.75) (end 123 97.75) (width 0.25) (layer "F.Cu") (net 6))
 (segment (start 123 97.75) (end 125 97.75) (width 0.25) (layer "F.Cu") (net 6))
 (segment (start 142.25 115) (end 142.25 118.75) (width 0.25) (layer "F.Cu") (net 6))
 (segment (start 125 97.75) (end 142.25 115) (width 0.25) (layer "F.Cu") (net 6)))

